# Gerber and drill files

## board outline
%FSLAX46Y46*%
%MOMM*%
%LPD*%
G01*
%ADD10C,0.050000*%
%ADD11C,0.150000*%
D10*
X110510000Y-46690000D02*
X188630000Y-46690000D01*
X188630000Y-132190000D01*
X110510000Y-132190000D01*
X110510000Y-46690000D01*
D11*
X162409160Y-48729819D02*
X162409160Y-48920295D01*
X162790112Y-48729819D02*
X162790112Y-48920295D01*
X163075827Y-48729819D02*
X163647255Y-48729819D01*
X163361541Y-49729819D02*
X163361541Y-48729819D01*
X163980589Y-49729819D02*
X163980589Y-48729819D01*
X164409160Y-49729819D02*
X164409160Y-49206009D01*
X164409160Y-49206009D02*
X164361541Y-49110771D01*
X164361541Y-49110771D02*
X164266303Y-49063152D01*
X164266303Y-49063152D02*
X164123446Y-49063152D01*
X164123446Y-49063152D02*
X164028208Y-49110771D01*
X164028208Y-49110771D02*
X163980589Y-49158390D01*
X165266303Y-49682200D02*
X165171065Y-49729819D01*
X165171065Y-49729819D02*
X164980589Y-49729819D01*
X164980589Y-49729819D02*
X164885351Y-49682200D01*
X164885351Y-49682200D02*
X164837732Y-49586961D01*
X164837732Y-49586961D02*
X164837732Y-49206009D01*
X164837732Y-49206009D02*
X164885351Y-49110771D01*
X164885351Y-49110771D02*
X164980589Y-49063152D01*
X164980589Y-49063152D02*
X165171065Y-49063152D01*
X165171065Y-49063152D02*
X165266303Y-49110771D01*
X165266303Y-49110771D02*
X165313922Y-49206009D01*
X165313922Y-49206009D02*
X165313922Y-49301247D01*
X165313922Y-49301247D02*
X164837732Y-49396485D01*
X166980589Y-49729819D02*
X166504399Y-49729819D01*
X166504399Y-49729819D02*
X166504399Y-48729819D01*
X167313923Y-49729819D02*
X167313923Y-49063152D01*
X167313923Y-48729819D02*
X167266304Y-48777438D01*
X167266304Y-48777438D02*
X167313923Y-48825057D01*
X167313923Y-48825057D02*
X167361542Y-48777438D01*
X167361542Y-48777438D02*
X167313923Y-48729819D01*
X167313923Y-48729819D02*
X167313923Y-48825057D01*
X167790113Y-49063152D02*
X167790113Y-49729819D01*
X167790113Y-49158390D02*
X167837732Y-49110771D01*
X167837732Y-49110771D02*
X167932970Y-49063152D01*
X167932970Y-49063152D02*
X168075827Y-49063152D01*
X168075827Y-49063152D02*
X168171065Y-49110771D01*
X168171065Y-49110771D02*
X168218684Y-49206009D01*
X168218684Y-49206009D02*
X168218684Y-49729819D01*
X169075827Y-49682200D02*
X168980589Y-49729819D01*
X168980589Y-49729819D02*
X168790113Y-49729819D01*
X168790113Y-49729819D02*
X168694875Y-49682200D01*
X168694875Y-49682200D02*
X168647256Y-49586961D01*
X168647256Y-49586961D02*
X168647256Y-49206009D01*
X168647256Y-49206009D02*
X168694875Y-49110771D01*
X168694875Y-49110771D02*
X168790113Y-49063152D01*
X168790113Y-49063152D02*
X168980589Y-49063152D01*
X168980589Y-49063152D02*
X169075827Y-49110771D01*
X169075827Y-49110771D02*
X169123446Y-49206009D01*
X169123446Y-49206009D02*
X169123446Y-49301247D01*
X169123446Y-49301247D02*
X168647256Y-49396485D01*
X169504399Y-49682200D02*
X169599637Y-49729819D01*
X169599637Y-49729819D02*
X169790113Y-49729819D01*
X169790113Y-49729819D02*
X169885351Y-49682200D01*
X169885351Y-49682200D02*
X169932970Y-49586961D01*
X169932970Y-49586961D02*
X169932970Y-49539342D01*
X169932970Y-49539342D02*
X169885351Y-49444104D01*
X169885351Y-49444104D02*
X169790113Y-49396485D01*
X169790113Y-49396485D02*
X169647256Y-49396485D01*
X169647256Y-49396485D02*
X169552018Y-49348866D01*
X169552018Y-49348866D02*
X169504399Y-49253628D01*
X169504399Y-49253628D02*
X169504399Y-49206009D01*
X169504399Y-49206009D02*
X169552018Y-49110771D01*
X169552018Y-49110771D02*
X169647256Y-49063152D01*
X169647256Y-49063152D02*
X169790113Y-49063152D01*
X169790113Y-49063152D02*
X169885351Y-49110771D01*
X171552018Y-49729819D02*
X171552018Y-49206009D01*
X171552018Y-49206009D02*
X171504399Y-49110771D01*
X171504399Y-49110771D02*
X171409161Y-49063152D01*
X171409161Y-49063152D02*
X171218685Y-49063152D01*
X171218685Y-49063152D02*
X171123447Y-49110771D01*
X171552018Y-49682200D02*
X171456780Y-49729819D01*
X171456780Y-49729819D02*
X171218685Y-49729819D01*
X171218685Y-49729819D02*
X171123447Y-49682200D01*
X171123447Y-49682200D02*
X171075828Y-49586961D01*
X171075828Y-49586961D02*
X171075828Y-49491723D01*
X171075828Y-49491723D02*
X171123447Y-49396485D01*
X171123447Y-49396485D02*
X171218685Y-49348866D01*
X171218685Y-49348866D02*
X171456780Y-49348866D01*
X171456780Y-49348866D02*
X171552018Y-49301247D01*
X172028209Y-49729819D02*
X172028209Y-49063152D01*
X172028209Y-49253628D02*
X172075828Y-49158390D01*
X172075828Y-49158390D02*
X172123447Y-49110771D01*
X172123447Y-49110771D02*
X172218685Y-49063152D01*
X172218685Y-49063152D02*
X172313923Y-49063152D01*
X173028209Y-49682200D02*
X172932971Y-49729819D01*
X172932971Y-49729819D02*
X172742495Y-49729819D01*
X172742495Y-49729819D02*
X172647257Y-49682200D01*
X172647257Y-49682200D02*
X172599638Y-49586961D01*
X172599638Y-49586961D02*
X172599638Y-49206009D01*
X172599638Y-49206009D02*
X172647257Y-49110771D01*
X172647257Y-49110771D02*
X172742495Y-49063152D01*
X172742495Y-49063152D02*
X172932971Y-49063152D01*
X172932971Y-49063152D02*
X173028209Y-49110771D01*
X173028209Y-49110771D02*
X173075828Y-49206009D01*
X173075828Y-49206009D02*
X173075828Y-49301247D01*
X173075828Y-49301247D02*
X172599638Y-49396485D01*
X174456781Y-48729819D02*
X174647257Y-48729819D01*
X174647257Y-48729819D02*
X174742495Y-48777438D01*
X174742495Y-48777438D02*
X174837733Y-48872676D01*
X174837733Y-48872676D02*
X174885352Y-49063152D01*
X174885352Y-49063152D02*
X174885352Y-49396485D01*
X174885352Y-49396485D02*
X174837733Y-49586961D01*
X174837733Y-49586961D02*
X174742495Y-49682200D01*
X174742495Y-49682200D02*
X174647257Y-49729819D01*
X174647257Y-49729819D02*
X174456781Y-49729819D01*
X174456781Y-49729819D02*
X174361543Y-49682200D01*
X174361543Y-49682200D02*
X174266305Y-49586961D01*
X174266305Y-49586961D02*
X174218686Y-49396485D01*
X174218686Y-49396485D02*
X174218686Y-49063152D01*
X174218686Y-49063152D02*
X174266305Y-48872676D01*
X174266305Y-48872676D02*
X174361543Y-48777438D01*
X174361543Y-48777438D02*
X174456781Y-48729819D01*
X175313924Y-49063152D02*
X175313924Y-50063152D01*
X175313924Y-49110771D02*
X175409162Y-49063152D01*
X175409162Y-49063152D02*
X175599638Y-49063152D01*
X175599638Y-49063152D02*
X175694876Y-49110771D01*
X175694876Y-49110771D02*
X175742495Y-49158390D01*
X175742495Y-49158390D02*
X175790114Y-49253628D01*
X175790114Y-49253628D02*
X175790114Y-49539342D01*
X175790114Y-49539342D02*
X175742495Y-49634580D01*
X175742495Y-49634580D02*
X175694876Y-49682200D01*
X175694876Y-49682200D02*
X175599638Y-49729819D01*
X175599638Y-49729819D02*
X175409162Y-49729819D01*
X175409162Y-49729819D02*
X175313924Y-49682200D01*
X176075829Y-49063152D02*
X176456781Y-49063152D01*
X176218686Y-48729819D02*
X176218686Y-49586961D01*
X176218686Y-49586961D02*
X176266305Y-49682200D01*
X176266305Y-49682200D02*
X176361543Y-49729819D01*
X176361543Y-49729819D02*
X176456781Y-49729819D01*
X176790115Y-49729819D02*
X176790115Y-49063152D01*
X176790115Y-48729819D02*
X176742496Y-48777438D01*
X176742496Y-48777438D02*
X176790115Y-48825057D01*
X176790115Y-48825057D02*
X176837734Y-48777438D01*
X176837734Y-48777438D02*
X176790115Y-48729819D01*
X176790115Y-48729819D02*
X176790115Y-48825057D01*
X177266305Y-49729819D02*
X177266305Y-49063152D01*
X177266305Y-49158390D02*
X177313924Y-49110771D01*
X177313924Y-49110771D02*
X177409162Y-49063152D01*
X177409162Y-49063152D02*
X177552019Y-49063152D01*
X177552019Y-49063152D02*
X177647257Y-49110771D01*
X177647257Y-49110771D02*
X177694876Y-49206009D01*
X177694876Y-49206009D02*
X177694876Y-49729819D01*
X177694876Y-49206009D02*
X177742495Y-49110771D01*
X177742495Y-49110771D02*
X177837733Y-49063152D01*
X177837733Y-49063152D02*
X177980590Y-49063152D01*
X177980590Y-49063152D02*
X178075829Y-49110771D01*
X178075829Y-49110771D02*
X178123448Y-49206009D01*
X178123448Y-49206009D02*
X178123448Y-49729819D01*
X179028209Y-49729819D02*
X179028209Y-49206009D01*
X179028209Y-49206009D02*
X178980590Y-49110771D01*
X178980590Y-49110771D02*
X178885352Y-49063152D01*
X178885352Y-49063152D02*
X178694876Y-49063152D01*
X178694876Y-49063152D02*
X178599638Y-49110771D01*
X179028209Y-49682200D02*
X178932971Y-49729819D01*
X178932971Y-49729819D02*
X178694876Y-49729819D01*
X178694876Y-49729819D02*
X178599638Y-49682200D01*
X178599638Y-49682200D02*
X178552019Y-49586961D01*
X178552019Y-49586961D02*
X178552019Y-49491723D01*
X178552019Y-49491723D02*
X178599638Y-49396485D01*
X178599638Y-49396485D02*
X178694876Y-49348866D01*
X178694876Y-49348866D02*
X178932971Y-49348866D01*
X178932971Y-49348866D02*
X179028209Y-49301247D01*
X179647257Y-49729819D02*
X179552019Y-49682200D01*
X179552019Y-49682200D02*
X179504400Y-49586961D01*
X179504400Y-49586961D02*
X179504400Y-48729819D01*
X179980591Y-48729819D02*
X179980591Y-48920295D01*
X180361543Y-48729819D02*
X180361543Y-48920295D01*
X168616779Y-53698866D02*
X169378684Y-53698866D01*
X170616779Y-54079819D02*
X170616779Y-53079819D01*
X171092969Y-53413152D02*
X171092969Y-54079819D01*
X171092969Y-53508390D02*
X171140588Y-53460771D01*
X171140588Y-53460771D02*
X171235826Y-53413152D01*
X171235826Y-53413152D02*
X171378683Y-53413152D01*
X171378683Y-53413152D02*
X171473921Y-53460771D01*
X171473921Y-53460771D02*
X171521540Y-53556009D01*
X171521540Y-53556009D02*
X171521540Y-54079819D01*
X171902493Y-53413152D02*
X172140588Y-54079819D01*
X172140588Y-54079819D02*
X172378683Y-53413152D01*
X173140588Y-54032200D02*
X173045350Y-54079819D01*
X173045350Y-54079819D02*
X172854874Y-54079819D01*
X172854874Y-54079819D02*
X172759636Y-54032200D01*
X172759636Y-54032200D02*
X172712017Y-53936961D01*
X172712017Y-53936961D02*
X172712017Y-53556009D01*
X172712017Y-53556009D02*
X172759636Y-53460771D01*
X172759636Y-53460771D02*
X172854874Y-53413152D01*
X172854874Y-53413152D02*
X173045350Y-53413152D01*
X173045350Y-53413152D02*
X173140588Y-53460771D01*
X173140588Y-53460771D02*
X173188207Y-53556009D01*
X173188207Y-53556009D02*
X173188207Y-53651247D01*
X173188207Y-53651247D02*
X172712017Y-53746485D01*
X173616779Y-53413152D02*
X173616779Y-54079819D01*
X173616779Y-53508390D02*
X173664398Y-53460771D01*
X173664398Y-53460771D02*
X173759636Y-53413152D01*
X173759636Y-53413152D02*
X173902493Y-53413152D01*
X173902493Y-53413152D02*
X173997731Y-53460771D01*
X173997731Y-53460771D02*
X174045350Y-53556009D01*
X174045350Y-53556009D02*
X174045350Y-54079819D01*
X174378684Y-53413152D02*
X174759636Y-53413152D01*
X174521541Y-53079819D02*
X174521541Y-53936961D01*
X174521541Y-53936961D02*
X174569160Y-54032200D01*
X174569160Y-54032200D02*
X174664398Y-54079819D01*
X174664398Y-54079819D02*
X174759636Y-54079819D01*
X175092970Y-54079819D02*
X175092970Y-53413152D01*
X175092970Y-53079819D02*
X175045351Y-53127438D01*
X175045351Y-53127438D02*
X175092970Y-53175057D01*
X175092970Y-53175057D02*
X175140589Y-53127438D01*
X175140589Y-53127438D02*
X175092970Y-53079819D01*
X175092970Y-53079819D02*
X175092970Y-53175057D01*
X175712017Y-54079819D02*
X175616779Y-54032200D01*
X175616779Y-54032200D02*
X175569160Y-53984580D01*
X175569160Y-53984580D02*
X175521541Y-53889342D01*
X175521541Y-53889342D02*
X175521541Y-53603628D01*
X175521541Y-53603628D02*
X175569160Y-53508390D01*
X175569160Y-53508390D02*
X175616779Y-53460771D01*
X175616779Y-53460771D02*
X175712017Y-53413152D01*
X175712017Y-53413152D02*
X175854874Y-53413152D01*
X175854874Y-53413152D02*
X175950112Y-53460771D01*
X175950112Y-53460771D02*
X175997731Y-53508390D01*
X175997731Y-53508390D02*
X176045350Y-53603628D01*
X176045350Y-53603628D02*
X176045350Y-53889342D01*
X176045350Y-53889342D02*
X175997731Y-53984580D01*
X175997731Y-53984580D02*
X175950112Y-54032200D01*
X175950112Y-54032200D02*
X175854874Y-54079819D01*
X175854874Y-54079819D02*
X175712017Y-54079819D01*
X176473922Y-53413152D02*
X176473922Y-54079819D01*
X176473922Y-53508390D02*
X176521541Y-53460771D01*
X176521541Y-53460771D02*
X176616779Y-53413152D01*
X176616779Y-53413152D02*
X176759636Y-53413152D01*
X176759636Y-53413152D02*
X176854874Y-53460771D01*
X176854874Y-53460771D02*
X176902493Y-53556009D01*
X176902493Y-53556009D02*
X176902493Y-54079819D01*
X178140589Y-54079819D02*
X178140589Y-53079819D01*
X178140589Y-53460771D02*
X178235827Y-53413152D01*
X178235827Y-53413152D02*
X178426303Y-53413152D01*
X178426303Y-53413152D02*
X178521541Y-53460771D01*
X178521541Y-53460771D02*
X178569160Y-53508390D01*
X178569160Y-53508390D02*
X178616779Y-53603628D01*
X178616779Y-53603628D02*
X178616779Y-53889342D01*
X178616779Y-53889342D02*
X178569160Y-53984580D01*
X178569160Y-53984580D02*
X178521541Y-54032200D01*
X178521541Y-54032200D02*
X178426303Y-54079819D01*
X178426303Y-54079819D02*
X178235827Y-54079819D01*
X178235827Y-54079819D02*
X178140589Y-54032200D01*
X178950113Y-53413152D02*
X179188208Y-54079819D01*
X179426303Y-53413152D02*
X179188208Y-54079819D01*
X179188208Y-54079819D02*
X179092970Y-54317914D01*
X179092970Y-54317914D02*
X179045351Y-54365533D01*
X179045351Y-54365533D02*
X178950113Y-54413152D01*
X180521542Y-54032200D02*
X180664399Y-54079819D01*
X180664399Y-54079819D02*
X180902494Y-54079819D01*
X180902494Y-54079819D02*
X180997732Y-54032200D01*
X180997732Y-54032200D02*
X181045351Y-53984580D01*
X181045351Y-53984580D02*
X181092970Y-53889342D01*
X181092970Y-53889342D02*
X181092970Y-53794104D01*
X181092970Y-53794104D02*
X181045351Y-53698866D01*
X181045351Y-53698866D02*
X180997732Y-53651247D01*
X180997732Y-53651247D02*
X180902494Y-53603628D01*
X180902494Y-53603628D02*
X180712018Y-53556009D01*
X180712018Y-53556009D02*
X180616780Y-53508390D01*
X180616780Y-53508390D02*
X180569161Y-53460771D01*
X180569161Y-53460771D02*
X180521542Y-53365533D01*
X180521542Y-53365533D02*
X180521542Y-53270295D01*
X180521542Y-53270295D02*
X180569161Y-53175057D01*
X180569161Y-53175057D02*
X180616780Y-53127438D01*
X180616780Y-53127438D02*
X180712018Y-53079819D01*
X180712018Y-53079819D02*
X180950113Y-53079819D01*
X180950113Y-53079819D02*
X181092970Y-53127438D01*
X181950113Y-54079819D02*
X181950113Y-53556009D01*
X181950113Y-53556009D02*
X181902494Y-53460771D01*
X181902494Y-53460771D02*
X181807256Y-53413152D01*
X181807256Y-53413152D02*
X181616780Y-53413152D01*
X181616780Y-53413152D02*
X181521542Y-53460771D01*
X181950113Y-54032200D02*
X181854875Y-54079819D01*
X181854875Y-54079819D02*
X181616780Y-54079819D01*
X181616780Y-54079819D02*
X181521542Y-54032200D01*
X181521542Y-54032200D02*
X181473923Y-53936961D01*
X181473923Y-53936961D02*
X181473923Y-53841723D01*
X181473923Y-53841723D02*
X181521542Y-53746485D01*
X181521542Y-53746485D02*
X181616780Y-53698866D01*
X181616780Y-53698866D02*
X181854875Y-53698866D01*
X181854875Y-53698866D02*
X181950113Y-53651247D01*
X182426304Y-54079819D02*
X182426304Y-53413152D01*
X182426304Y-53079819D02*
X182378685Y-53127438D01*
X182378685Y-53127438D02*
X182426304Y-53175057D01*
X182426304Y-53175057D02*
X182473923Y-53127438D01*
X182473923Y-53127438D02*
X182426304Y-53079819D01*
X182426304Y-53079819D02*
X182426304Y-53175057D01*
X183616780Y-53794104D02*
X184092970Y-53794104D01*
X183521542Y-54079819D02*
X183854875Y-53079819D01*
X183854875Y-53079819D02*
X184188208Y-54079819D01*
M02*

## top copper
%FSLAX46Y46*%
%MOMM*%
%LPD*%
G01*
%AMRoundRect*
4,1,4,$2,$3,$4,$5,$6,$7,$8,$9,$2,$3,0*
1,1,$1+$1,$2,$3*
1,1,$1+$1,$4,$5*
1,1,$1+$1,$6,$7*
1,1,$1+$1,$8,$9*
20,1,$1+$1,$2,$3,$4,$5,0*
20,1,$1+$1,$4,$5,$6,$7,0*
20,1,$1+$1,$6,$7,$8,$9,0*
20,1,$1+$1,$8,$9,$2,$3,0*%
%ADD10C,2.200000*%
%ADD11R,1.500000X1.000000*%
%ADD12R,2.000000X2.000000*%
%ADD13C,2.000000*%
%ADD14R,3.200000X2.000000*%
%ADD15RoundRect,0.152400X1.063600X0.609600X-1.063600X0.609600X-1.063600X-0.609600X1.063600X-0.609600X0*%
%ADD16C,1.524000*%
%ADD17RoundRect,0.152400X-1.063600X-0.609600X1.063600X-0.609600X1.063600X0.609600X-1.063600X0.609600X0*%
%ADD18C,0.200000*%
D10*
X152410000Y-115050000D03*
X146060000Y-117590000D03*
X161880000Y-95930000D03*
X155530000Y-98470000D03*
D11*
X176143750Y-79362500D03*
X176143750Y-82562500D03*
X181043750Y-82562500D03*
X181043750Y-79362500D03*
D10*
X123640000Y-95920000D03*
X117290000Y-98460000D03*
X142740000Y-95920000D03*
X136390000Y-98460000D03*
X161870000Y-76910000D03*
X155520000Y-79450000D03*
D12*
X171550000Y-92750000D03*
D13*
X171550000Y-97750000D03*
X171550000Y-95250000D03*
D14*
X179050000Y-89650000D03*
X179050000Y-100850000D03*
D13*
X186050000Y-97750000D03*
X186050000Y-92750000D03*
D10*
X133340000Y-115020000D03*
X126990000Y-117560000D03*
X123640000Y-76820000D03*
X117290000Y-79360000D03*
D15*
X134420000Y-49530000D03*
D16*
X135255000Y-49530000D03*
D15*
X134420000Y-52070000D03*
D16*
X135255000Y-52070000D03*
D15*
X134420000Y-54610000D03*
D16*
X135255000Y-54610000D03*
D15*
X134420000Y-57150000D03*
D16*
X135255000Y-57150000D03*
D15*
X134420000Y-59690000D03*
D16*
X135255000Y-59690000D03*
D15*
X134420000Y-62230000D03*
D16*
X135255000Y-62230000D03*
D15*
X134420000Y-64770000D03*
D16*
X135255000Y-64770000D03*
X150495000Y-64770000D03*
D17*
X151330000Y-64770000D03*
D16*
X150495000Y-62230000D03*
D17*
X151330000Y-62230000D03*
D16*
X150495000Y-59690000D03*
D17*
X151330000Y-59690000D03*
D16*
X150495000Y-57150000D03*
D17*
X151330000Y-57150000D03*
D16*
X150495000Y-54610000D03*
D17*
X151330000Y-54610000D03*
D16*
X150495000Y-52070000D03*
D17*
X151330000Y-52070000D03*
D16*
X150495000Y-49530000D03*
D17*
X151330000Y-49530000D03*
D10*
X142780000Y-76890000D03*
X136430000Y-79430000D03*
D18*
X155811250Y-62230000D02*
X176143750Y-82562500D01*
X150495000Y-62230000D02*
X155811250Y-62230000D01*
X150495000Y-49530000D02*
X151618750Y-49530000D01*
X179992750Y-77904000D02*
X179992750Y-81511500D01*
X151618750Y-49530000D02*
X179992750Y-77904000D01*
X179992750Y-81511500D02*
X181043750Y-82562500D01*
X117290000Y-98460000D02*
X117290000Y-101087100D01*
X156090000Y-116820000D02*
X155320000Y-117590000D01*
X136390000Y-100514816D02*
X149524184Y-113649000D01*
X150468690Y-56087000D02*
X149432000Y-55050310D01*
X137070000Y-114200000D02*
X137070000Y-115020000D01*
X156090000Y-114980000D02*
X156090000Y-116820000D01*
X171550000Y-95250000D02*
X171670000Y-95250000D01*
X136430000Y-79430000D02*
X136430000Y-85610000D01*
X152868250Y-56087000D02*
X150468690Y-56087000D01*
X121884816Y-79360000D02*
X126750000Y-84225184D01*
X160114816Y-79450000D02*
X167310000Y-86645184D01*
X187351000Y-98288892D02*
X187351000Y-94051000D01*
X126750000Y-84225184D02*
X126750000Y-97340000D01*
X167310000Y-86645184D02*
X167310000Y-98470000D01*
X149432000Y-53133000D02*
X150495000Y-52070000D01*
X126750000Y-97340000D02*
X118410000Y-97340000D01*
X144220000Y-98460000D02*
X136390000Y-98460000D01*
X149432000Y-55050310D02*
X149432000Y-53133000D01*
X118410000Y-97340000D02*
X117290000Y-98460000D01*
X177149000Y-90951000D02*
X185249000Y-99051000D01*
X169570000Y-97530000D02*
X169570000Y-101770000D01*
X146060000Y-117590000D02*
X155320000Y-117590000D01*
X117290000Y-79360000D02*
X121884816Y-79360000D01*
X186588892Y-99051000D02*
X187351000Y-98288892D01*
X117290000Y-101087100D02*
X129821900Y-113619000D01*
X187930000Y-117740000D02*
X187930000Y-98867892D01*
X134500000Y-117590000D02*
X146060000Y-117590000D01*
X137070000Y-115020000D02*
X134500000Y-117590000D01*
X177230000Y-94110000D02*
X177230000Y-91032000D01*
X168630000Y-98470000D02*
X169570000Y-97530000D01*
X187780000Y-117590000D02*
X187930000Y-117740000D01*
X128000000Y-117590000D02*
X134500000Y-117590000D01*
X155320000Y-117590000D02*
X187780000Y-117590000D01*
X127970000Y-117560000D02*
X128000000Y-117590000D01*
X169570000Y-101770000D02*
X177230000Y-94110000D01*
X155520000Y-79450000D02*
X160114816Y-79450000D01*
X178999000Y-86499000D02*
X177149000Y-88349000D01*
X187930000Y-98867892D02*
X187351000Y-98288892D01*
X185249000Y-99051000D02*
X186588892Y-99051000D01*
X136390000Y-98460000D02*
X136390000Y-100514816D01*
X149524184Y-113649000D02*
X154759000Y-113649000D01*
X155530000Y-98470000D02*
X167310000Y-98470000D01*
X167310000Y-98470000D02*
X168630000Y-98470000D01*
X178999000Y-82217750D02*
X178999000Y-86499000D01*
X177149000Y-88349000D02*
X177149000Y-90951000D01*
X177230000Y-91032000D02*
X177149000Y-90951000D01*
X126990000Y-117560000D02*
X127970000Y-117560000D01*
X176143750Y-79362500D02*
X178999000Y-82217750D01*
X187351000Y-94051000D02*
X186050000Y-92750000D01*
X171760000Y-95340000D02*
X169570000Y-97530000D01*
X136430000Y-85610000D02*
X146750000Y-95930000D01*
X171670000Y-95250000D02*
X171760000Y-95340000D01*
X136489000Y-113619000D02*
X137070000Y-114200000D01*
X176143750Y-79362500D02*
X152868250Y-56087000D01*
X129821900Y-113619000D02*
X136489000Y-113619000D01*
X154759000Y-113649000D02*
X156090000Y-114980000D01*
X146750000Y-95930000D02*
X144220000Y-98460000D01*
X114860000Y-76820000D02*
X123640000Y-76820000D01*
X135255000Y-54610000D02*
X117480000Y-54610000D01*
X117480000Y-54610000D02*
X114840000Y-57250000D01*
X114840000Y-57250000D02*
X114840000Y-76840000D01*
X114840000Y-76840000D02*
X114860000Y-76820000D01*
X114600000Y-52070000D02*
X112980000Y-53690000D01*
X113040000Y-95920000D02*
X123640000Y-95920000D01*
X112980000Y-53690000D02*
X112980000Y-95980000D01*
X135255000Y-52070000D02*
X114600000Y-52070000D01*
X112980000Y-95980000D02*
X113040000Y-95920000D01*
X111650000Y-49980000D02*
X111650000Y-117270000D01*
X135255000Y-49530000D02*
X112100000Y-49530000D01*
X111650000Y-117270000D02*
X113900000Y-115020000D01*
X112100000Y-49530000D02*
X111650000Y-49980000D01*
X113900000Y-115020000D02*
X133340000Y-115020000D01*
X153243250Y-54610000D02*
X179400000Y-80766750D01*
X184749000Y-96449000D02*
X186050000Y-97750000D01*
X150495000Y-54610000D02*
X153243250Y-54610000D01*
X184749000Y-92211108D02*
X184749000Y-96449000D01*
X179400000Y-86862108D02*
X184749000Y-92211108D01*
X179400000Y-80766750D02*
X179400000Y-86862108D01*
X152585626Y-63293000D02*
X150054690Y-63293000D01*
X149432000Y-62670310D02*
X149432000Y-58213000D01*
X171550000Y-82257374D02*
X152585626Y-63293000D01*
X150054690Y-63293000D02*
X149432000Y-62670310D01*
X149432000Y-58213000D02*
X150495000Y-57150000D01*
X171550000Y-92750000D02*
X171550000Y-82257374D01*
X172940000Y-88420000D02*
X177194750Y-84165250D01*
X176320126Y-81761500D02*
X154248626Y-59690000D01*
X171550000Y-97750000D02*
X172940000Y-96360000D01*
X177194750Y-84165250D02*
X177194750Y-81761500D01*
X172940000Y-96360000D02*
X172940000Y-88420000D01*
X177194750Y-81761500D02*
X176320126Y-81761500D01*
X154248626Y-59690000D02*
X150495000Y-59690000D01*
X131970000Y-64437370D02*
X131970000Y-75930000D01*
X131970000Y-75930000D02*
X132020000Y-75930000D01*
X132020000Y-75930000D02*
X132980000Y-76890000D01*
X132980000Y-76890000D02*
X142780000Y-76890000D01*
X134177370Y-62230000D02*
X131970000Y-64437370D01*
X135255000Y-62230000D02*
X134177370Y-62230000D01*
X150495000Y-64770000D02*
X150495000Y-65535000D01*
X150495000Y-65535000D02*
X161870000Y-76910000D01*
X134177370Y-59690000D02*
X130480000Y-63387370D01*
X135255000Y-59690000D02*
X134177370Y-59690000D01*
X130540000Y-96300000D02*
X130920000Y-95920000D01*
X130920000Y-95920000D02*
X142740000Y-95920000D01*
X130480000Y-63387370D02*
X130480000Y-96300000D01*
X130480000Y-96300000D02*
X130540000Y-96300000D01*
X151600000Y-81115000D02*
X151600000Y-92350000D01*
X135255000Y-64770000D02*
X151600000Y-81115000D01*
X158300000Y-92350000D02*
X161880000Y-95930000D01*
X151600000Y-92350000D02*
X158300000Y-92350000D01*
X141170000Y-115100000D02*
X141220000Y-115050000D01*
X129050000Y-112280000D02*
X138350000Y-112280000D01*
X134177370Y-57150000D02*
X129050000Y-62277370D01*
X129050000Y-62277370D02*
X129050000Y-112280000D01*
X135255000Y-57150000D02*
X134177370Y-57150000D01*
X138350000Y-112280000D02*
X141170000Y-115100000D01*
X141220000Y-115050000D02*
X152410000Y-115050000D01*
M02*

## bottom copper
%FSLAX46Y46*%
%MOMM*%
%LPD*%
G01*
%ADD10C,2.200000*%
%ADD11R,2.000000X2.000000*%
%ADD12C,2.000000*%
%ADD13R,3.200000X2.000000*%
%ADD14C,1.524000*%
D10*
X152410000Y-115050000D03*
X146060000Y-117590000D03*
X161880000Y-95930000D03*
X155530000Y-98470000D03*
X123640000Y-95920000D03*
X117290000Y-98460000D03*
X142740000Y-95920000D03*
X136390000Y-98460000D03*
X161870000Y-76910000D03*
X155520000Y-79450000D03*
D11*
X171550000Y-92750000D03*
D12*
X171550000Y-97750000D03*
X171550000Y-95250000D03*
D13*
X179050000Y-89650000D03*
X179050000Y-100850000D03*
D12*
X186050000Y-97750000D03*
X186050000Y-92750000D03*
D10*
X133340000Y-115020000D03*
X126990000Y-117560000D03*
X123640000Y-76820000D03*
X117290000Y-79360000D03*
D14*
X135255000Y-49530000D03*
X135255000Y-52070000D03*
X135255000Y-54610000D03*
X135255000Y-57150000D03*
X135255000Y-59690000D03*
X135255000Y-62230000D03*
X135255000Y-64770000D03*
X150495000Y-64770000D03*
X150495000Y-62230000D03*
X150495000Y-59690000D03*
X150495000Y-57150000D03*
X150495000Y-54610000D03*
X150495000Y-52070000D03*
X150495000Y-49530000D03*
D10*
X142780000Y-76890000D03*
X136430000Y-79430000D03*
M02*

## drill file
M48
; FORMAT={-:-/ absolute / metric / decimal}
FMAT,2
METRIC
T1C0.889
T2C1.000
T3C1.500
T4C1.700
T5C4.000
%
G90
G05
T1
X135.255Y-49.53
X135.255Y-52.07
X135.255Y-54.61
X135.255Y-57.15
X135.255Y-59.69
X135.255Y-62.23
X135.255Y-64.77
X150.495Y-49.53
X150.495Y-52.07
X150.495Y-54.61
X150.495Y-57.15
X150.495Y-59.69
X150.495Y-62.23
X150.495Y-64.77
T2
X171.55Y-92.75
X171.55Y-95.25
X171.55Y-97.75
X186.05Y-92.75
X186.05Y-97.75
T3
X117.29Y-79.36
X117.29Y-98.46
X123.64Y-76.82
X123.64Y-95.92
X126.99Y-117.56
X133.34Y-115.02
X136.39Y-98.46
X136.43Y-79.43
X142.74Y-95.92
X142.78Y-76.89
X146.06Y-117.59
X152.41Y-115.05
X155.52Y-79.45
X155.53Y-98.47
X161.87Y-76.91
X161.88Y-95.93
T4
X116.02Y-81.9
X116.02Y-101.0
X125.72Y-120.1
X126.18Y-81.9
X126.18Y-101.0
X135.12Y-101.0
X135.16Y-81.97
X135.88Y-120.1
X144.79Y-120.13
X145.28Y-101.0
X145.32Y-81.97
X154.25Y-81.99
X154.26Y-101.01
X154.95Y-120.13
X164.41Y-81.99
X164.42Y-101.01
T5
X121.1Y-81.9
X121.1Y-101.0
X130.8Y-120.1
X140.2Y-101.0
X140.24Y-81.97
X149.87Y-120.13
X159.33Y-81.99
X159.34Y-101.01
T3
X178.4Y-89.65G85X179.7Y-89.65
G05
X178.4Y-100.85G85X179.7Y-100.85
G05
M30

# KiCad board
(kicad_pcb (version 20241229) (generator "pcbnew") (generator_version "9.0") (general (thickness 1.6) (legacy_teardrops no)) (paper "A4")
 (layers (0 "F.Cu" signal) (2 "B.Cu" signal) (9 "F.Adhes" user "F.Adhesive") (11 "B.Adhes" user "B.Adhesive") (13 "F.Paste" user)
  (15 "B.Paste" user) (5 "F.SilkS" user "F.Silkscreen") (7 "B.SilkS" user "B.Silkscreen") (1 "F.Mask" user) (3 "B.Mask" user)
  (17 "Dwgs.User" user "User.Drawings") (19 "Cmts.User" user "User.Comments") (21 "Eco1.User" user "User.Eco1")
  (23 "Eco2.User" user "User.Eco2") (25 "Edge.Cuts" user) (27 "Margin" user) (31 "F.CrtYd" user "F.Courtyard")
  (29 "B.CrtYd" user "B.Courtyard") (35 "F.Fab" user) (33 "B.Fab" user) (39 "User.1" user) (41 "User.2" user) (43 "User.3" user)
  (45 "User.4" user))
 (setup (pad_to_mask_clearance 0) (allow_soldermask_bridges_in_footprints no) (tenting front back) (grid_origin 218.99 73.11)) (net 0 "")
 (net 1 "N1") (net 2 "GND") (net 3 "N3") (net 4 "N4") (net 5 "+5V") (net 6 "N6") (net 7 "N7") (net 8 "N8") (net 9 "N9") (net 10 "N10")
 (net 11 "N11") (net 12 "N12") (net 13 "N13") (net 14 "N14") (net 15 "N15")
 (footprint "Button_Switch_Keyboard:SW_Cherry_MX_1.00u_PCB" (layer "F.Cu") (at 152.41 115.05)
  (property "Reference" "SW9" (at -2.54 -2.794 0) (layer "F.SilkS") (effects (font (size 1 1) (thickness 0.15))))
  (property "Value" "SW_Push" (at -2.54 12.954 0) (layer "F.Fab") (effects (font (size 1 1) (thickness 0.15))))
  (pad "" np_thru_hole circle (at -7.62 5.08) (size 1.7 1.7) (drill 1.7) (layers "*.Cu" "*.Mask"))
  (pad "" np_thru_hole circle (at -2.54 5.08) (size 4 4) (drill 4) (layers "*.Cu" "*.Mask"))
  (pad "" np_thru_hole circle (at 2.54 5.08) (size 1.7 1.7) (drill 1.7) (layers "*.Cu" "*.Mask"))
  (pad "1" thru_hole circle (at 0 0) (size 2.2 2.2) (drill 1.5) (layers "*.Cu" "*.Mask") (remove_unused_layers no) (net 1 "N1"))
  (pad "2" thru_hole circle (at -6.35 2.54) (size 2.2 2.2) (drill 1.5) (layers "*.Cu" "*.Mask") (remove_unused_layers no) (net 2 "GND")))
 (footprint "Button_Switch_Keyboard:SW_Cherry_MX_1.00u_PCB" (layer "F.Cu") (at 161.88 95.93)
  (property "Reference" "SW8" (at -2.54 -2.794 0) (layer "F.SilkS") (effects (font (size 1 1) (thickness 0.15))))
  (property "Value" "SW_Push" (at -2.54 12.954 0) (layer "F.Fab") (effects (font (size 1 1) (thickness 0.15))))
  (pad "" np_thru_hole circle (at -7.62 5.08) (size 1.7 1.7) (drill 1.7) (layers "*.Cu" "*.Mask"))
  (pad "" np_thru_hole circle (at -2.54 5.08) (size 4 4) (drill 4) (layers "*.Cu" "*.Mask"))
  (pad "" np_thru_hole circle (at 2.54 5.08) (size 1.7 1.7) (drill 1.7) (layers "*.Cu" "*.Mask"))
  (pad "1" thru_hole circle (at 0 0) (size 2.2 2.2) (drill 1.5) (layers "*.Cu" "*.Mask") (remove_unused_layers no) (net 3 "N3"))
  (pad "2" thru_hole circle (at -6.35 2.54) (size 2.2 2.2) (drill 1.5) (layers "*.Cu" "*.Mask") (remove_unused_layers no) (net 2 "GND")))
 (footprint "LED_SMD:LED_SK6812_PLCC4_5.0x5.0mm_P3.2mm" (layer "F.Cu") (at 178.59375 80.9625)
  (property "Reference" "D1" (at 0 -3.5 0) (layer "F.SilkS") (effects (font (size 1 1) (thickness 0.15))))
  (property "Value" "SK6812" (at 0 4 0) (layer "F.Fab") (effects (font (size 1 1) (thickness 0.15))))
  (pad "1" smd rect (at -2.45 -1.6 180) (size 1.5 1) (layers "F.Cu" "F.Mask" "F.Paste") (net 2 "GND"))
  (pad "2" smd rect (at -2.45 1.6 180) (size 1.5 1) (layers "F.Cu" "F.Mask" "F.Paste") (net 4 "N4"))
  (pad "3" smd rect (at 2.45 1.6 180) (size 1.5 1) (layers "F.Cu" "F.Mask" "F.Paste") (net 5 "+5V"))
  (pad "4" smd rect (at 2.45 -1.6 180) (size 1.5 1) (layers "F.Cu" "F.Mask" "F.Paste") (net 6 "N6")))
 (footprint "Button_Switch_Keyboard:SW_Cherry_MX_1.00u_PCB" (layer "F.Cu") (at 123.64 95.92)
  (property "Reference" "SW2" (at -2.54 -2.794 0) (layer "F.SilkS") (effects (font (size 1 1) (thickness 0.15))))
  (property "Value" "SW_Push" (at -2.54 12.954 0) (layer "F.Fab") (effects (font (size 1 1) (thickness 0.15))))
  (pad "" np_thru_hole circle (at -7.62 5.08) (size 1.7 1.7) (drill 1.7) (layers "*.Cu" "*.Mask"))
  (pad "" np_thru_hole circle (at -2.54 5.08) (size 4 4) (drill 4) (layers "*.Cu" "*.Mask"))
  (pad "" np_thru_hole circle (at 2.54 5.08) (size 1.7 1.7) (drill 1.7) (layers "*.Cu" "*.Mask"))
  (pad "1" thru_hole circle (at 0 0) (size 2.2 2.2) (drill 1.5) (layers "*.Cu" "*.Mask") (remove_unused_layers no) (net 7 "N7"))
  (pad "2" thru_hole circle (at -6.35 2.54) (size 2.2 2.2) (drill 1.5) (layers "*.Cu" "*.Mask") (remove_unused_layers no) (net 2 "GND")))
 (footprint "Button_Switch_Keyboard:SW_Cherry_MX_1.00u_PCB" (layer "F.Cu") (at 142.74 95.92)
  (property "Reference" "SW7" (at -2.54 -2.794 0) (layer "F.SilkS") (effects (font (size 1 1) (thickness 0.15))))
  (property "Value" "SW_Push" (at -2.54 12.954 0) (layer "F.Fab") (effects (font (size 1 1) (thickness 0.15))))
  (pad "" np_thru_hole circle (at -7.62 5.08) (size 1.7 1.7) (drill 1.7) (layers "*.Cu" "*.Mask"))
  (pad "" np_thru_hole circle (at -2.54 5.08) (size 4 4) (drill 4) (layers "*.Cu" "*.Mask"))
  (pad "" np_thru_hole circle (at 2.54 5.08) (size 1.7 1.7) (drill 1.7) (layers "*.Cu" "*.Mask"))
  (pad "1" thru_hole circle (at 0 0) (size 2.2 2.2) (drill 1.5) (layers "*.Cu" "*.Mask") (remove_unused_layers no) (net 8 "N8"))
  (pad "2" thru_hole circle (at -6.35 2.54) (size 2.2 2.2) (drill 1.5) (layers "*.Cu" "*.Mask") (remove_unused_layers no) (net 2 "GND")))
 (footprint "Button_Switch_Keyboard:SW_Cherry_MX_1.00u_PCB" (layer "F.Cu") (at 161.87 76.91)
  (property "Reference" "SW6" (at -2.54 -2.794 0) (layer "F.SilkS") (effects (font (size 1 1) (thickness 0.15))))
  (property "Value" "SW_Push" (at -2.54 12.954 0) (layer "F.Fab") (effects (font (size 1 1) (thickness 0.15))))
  (pad "" np_thru_hole circle (at -7.62 5.08) (size 1.7 1.7) (drill 1.7) (layers "*.Cu" "*.Mask"))
  (pad "" np_thru_hole circle (at -2.54 5.08) (size 4 4) (drill 4) (layers "*.Cu" "*.Mask"))
  (pad "" np_thru_hole circle (at 2.54 5.08) (size 1.7 1.7) (drill 1.7) (layers "*.Cu" "*.Mask"))
  (pad "1" thru_hole circle (at 0 0) (size 2.2 2.2) (drill 1.5) (layers "*.Cu" "*.Mask") (remove_unused_layers no) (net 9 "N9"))
  (pad "2" thru_hole circle (at -6.35 2.54) (size 2.2 2.2) (drill 1.5) (layers "*.Cu" "*.Mask") (remove_unused_layers no) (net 2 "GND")))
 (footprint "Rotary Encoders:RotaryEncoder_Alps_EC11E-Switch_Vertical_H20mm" (layer "F.Cu") (at 171.55 92.75)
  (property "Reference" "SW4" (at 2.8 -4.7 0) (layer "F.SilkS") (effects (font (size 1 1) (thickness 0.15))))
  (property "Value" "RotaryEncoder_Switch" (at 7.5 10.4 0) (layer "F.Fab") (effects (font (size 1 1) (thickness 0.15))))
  (pad "A" thru_hole rect (at 0 0) (size 2 2) (drill 1) (layers "*.Cu" "*.Mask") (remove_unused_layers no) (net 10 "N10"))
  (pad "B" thru_hole circle (at 0 5) (size 2 2) (drill 1) (layers "*.Cu" "*.Mask") (remove_unused_layers no) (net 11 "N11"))
  (pad "C" thru_hole circle (at 0 2.5) (size 2 2) (drill 1) (layers "*.Cu" "*.Mask") (remove_unused_layers no) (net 2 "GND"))
  (pad "MP" thru_hole rect (at 7.5 -3.1) (size 3.2 2) (drill oval 2.8 1.5) (layers "*.Cu" "*.Mask") (remove_unused_layers no))
  (pad "MP" thru_hole rect (at 7.5 8.1) (size 3.2 2) (drill oval 2.8 1.5) (layers "*.Cu" "*.Mask") (remove_unused_layers no))
  (pad "S1" thru_hole circle (at 14.5 5) (size 2 2) (drill 1) (layers "*.Cu" "*.Mask") (remove_unused_layers no) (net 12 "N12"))
  (pad "S2" thru_hole circle (at 14.5 0) (size 2 2) (drill 1) (layers "*.Cu" "*.Mask") (remove_unused_layers no) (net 2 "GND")))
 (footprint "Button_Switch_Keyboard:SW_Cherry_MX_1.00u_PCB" (layer "F.Cu") (at 133.34 115.02)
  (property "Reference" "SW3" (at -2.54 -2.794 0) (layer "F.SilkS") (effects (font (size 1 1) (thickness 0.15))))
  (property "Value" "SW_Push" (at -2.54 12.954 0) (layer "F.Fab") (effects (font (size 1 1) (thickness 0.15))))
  (pad "" np_thru_hole circle (at -7.62 5.08) (size 1.7 1.7) (drill 1.7) (layers "*.Cu" "*.Mask"))
  (pad "" np_thru_hole circle (at -2.54 5.08) (size 4 4) (drill 4) (layers "*.Cu" "*.Mask"))
  (pad "" np_thru_hole circle (at 2.54 5.08) (size 1.7 1.7) (drill 1.7) (layers "*.Cu" "*.Mask"))
  (pad "1" thru_hole circle (at 0 0) (size 2.2 2.2) (drill 1.5) (layers "*.Cu" "*.Mask") (remove_unused_layers no) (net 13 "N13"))
  (pad "2" thru_hole circle (at -6.35 2.54) (size 2.2 2.2) (drill 1.5) (layers "*.Cu" "*.Mask") (remove_unused_layers no) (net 2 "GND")))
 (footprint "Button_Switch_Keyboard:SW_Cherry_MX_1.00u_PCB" (layer "F.Cu") (at 123.64 76.82)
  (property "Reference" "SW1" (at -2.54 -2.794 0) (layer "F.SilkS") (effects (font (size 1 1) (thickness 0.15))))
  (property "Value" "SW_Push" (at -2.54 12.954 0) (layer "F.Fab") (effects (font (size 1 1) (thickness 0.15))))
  (pad "" np_thru_hole circle (at -7.62 5.08) (size 1.7 1.7) (drill 1.7) (layers "*.Cu" "*.Mask"))
  (pad "" np_thru_hole circle (at -2.54 5.08) (size 4 4) (drill 4) (layers "*.Cu" "*.Mask"))
  (pad "" np_thru_hole circle (at 2.54 5.08) (size 1.7 1.7) (drill 1.7) (layers "*.Cu" "*.Mask"))
  (pad "1" thru_hole circle (at 0 0) (size 2.2 2.2) (drill 1.5) (layers "*.Cu" "*.Mask") (remove_unused_layers no) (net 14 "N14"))
  (pad "2" thru_hole circle (at -6.35 2.54) (size 2.2 2.2) (drill 1.5) (layers "*.Cu" "*.Mask") (remove_unused_layers no) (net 2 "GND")))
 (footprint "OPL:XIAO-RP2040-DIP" (layer "F.Cu") (at 142.875 57.15)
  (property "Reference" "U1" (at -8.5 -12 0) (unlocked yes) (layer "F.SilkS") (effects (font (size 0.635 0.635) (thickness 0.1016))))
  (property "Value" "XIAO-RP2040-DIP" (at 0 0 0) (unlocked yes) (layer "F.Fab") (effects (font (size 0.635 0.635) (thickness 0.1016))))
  (pad "1" smd roundrect (at -8.455 -7.62 180) (size 2.432 1.524) (layers "F.Cu" "F.Mask") (roundrect_rratio 0.1) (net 13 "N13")
   (thermal_bridge_angle 45))
  (pad "1" thru_hole circle (at -7.62 -7.62 180) (size 1.524 1.524) (drill 0.889) (layers "*.Cu" "*.Mask") (remove_unused_layers no)
   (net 13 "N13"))
  (pad "2" smd roundrect (at -8.455 -5.08 180) (size 2.432 1.524) (layers "F.Cu" "F.Mask") (roundrect_rratio 0.1) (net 7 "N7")
   (thermal_bridge_angle 45))
  (pad "2" thru_hole circle (at -7.62 -5.08 180) (size 1.524 1.524) (drill 0.889) (layers "*.Cu" "*.Mask") (remove_unused_layers no)
   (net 7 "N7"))
  (pad "3" smd roundrect (at -8.455 -2.54 180) (size 2.432 1.524) (layers "F.Cu" "F.Mask") (roundrect_rratio 0.1) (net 14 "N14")
   (thermal_bridge_angle 45))
  (pad "3" thru_hole circle (at -7.62 -2.54 180) (size 1.524 1.524) (drill 0.889) (layers "*.Cu" "*.Mask") (remove_unused_layers no)
   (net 14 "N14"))
  (pad "4" smd roundrect (at -8.455 0 180) (size 2.432 1.524) (layers "F.Cu" "F.Mask") (roundrect_rratio 0.1) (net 1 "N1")
   (thermal_bridge_angle 45))
  (pad "4" thru_hole circle (at -7.62 0 180) (size 1.524 1.524) (drill 0.889) (layers "*.Cu" "*.Mask") (remove_unused_layers no)
   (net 1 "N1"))
  (pad "5" smd roundrect (at -8.455 2.54 180) (size 2.432 1.524) (layers "F.Cu" "F.Mask") (roundrect_rratio 0.1) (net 8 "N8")
   (thermal_bridge_angle 45))
  (pad "5" thru_hole circle (at -7.62 2.54 180) (size 1.524 1.524) (drill 0.889) (layers "*.Cu" "*.Mask") (remove_unused_layers no)
   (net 8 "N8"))
  (pad "6" smd roundrect (at -8.455 5.08 180) (size 2.432 1.524) (layers "F.Cu" "F.Mask") (roundrect_rratio 0.1) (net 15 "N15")
   (thermal_bridge_angle 45))
  (pad "6" thru_hole circle (at -7.62 5.08 180) (size 1.524 1.524) (drill 0.889) (layers "*.Cu" "*.Mask") (remove_unused_layers no)
   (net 15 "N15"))
  (pad "7" smd roundrect (at -8.455 7.62 180) (size 2.432 1.524) (layers "F.Cu" "F.Mask") (roundrect_rratio 0.1) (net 3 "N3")
   (thermal_bridge_angle 45))
  (pad "7" thru_hole circle (at -7.62 7.62 180) (size 1.524 1.524) (drill 0.889) (layers "*.Cu" "*.Mask") (remove_unused_layers no)
   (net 3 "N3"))
  (pad "8" thru_hole circle (at 7.62 7.62) (size 1.524 1.524) (drill 0.889) (layers "*.Cu" "*.Mask") (remove_unused_layers no) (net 9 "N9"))
  (pad "8" smd roundrect (at 8.455 7.62) (size 2.432 1.524) (layers "F.Cu" "F.Mask") (roundrect_rratio 0.1) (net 9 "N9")
   (thermal_bridge_angle 45))
  (pad "9" thru_hole circle (at 7.62 5.08) (size 1.524 1.524) (drill 0.889) (layers "*.Cu" "*.Mask") (remove_unused_layers no) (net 4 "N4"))
  (pad "9" smd roundrect (at 8.455 5.08) (size 2.432 1.524) (layers "F.Cu" "F.Mask") (roundrect_rratio 0.1) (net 4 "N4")
   (thermal_bridge_angle 45))
  (pad "10" thru_hole circle (at 7.62 2.54) (size 1.524 1.524) (drill 0.889) (layers "*.Cu" "*.Mask") (remove_unused_layers no)
   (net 11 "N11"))
  (pad "10" smd roundrect (at 8.455 2.54) (size 2.432 1.524) (layers "F.Cu" "F.Mask") (roundrect_rratio 0.1) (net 11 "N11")
   (thermal_bridge_angle 45))
  (pad "11" thru_hole circle (at 7.62 0) (size 1.524 1.524) (drill 0.889) (layers "*.Cu" "*.Mask") (remove_unused_layers no) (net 10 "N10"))
  (pad "11" smd roundrect (at 8.455 0) (size 2.432 1.524) (layers "F.Cu" "F.Mask") (roundrect_rratio 0.1) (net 10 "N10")
   (thermal_bridge_angle 45))
  (pad "12" thru_hole circle (at 7.62 -2.54) (size 1.524 1.524) (drill 0.889) (layers "*.Cu" "*.Mask") (remove_unused_layers no)
   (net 12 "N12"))
  (pad "12" smd roundrect (at 8.455 -2.54) (size 2.432 1.524) (layers "F.Cu" "F.Mask") (roundrect_rratio 0.1) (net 12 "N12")
   (thermal_bridge_angle 45))
  (pad "13" thru_hole circle (at 7.62 -5.08) (size 1.524 1.524) (drill 0.889) (layers "*.Cu" "*.Mask") (remove_unused_layers no)
   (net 2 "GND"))
  (pad "13" smd roundrect (at 8.455 -5.08) (size 2.432 1.524) (layers "F.Cu" "F.Mask") (roundrect_rratio 0.1) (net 2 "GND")
   (thermal_bridge_angle 45))
  (pad "14" thru_hole circle (at 7.62 -7.62) (size 1.524 1.524) (drill 0.889) (layers "*.Cu" "*.Mask") (remove_unused_layers no)
   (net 5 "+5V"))
  (pad "14" smd roundrect (at 8.455 -7.62) (size 2.432 1.524) (layers "F.Cu" "F.Mask") (roundrect_rratio 0.1) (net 5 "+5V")
   (thermal_bridge_angle 45)))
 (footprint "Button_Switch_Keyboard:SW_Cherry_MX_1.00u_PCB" (layer "F.Cu") (at 142.78 76.89)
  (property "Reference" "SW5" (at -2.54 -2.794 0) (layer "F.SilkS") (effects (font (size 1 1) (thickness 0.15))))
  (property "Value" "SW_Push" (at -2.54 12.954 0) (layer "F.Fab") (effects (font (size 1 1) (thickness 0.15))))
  (pad "" np_thru_hole circle (at -7.62 5.08) (size 1.7 1.7) (drill 1.7) (layers "*.Cu" "*.Mask"))
  (pad "" np_thru_hole circle (at -2.54 5.08) (size 4 4) (drill 4) (layers "*.Cu" "*.Mask"))
  (pad "" np_thru_hole circle (at 2.54 5.08) (size 1.7 1.7) (drill 1.7) (layers "*.Cu" "*.Mask"))
  (pad "1" thru_hole circle (at 0 0) (size 2.2 2.2) (drill 1.5) (layers "*.Cu" "*.Mask") (remove_unused_layers no) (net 15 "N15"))
  (pad "2" thru_hole circle (at -6.35 2.54) (size 2.2 2.2) (drill 1.5) (layers "*.Cu" "*.Mask") (remove_unused_layers no) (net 2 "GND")))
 (gr_rect (start 110.51 46.69) (end 188.63 132.19) (stroke (width 0.05) (type default)) (fill no) (layer "Edge.Cuts"))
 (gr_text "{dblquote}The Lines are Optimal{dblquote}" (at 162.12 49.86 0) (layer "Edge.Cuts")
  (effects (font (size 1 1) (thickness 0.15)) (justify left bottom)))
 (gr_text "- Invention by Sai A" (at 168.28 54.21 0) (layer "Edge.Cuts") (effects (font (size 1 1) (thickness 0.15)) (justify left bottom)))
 (segment (start 155.81125 62.23) (end 176.14375 82.5625) (width 0.2) (layer "F.Cu") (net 4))
 (segment (start 150.495 62.23) (end 155.81125 62.23) (width 0.2) (layer "F.Cu") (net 4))
 (segment (start 150.495 49.53) (end 151.61875 49.53) (width 0.2) (layer "F.Cu") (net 5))
 (segment (start 179.99275 77.904) (end 179.99275 81.5115) (width 0.2) (layer "F.Cu") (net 5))
 (segment (start 151.61875 49.53) (end 179.99275 77.904) (width 0.2) (layer "F.Cu") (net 5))
 (segment (start 179.99275 81.5115) (end 181.04375 82.5625) (width 0.2) (layer "F.Cu") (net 5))
 (segment (start 117.29 98.46) (end 117.29 101.0871) (width 0.2) (layer "F.Cu") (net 2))
 (segment (start 156.09 116.82) (end 155.32 117.59) (width 0.2) (layer "F.Cu") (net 2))
 (segment (start 136.39 100.514816) (end 149.524184 113.649) (width 0.2) (layer "F.Cu") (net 2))
 (segment (start 150.46869 56.087) (end 149.432 55.05031) (width 0.2) (layer "F.Cu") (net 2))
 (segment (start 137.07 114.2) (end 137.07 115.02) (width 0.2) (layer "F.Cu") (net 2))
 (segment (start 156.09 114.98) (end 156.09 116.82) (width 0.2) (layer "F.Cu") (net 2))
 (segment (start 171.55 95.25) (end 171.67 95.25) (width 0.2) (layer "F.Cu") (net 2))
 (segment (start 136.43 79.43) (end 136.43 85.61) (width 0.2) (layer "F.Cu") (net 2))
 (segment (start 152.86825 56.087) (end 150.46869 56.087) (width 0.2) (layer "F.Cu") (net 2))
 (segment (start 121.884816 79.36) (end 126.75 84.225184) (width 0.2) (layer "F.Cu") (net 2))
 (segment (start 160.114816 79.45) (end 167.31 86.645184) (width 0.2) (layer "F.Cu") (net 2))
 (segment (start 187.351 98.288892) (end 187.351 94.051) (width 0.2) (layer "F.Cu") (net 2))
 (segment (start 126.75 84.225184) (end 126.75 97.34) (width 0.2) (layer "F.Cu") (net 2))
 (segment (start 167.31 86.645184) (end 167.31 98.47) (width 0.2) (layer "F.Cu") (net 2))
 (segment (start 149.432 53.133) (end 150.495 52.07) (width 0.2) (layer "F.Cu") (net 2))
 (segment (start 126.75 97.34) (end 118.41 97.34) (width 0.2) (layer "F.Cu") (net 2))
 (segment (start 144.22 98.46) (end 136.39 98.46) (width 0.2) (layer "F.Cu") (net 2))
 (segment (start 149.432 55.05031) (end 149.432 53.133) (width 0.2) (layer "F.Cu") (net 2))
 (segment (start 118.41 97.34) (end 117.29 98.46) (width 0.2) (layer "F.Cu") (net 2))
 (segment (start 177.149 90.951) (end 185.249 99.051) (width 0.2) (layer "F.Cu") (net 2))
 (segment (start 169.57 97.53) (end 169.57 101.77) (width 0.2) (layer "F.Cu") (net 2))
 (segment (start 146.06 117.59) (end 155.32 117.59) (width 0.2) (layer "F.Cu") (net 2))
 (segment (start 117.29 79.36) (end 121.884816 79.36) (width 0.2) (layer "F.Cu") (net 2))
 (segment (start 186.588892 99.051) (end 187.351 98.288892) (width 0.2) (layer "F.Cu") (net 2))
 (segment (start 117.29 101.0871) (end 129.8219 113.619) (width 0.2) (layer "F.Cu") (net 2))
 (segment (start 187.93 117.74) (end 187.93 98.867892) (width 0.2) (layer "F.Cu") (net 2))
 (segment (start 134.5 117.59) (end 146.06 117.59) (width 0.2) (layer "F.Cu") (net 2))
 (segment (start 137.07 115.02) (end 134.5 117.59) (width 0.2) (layer "F.Cu") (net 2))
 (segment (start 177.23 94.11) (end 177.23 91.032) (width 0.2) (layer "F.Cu") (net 2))
 (segment (start 168.63 98.47) (end 169.57 97.53) (width 0.2) (layer "F.Cu") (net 2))
 (segment (start 187.78 117.59) (end 187.93 117.74) (width 0.2) (layer "F.Cu") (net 2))
 (segment (start 128 117.59) (end 134.5 117.59) (width 0.2) (layer "F.Cu") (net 2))
 (segment (start 155.32 117.59) (end 187.78 117.59) (width 0.2) (layer "F.Cu") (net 2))
 (segment (start 127.97 117.56) (end 128 117.59) (width 0.2) (layer "F.Cu") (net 2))
 (segment (start 169.57 101.77) (end 177.23 94.11) (width 0.2) (layer "F.Cu") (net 2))
 (segment (start 155.52 79.45) (end 160.114816 79.45) (width 0.2) (layer "F.Cu") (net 2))
 (segment (start 178.999 86.499) (end 177.149 88.349) (width 0.2) (layer "F.Cu") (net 2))
 (segment (start 187.93 98.867892) (end 187.351 98.288892) (width 0.2) (layer "F.Cu") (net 2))
 (segment (start 185.249 99.051) (end 186.588892 99.051) (width 0.2) (layer "F.Cu") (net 2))
 (segment (start 136.39 98.46) (end 136.39 100.514816) (width 0.2) (layer "F.Cu") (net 2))
 (segment (start 149.524184 113.649) (end 154.759 113.649) (width 0.2) (layer "F.Cu") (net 2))
 (segment (start 155.53 98.47) (end 167.31 98.47) (width 0.2) (layer "F.Cu") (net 2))
 (segment (start 167.31 98.47) (end 168.63 98.47) (width 0.2) (layer "F.Cu") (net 2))
 (segment (start 178.999 82.21775) (end 178.999 86.499) (width 0.2) (layer "F.Cu") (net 2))
 (segment (start 177.149 88.349) (end 177.149 90.951) (width 0.2) (layer "F.Cu") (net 2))
 (segment (start 177.23 91.032) (end 177.149 90.951) (width 0.2) (layer "F.Cu") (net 2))
 (segment (start 126.99 117.56) (end 127.97 117.56) (width 0.2) (layer "F.Cu") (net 2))
 (segment (start 176.14375 79.3625) (end 178.999 82.21775) (width 0.2) (layer "F.Cu") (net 2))
 (segment (start 187.351 94.051) (end 186.05 92.75) (width 0.2) (layer "F.Cu") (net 2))
 (segment (start 171.76 95.34) (end 169.57 97.53) (width 0.2) (layer "F.Cu") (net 2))
 (segment (start 136.43 85.61) (end 146.75 95.93) (width 0.2) (layer "F.Cu") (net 2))
 (segment (start 171.67 95.25) (end 171.76 95.34) (width 0.2) (layer "F.Cu") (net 2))
 (segment (start 136.489 113.619) (end 137.07 114.2) (width 0.2) (layer "F.Cu") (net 2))
 (segment (start 176.14375 79.3625) (end 152.86825 56.087) (width 0.2) (layer "F.Cu") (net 2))
 (segment (start 129.8219 113.619) (end 136.489 113.619) (width 0.2) (layer "F.Cu") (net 2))
 (segment (start 154.759 113.649) (end 156.09 114.98) (width 0.2) (layer "F.Cu") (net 2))
 (segment (start 146.75 95.93) (end 144.22 98.46) (width 0.2) (layer "F.Cu") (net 2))
 (segment (start 114.86 76.82) (end 123.64 76.82) (width 0.2) (layer "F.Cu") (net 14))
 (segment (start 135.255 54.61) (end 117.48 54.61) (width 0.2) (layer "F.Cu") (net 14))
 (segment (start 117.48 54.61) (end 114.84 57.25) (width 0.2) (layer "F.Cu") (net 14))
 (segment (start 114.84 57.25) (end 114.84 76.84) (width 0.2) (layer "F.Cu") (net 14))
 (segment (start 114.84 76.84) (end 114.86 76.82) (width 0.2) (layer "F.Cu") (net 14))
 (segment (start 114.6 52.07) (end 112.98 53.69) (width 0.2) (layer "F.Cu") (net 7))
 (segment (start 113.04 95.92) (end 123.64 95.92) (width 0.2) (layer "F.Cu") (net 7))
 (segment (start 112.98 53.69) (end 112.98 95.98) (width 0.2) (layer "F.Cu") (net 7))
 (segment (start 135.255 52.07) (end 114.6 52.07) (width 0.2) (layer "F.Cu") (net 7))
 (segment (start 112.98 95.98) (end 113.04 95.92) (width 0.2) (layer "F.Cu") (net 7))
 (segment (start 111.65 49.98) (end 111.65 117.27) (width 0.2) (layer "F.Cu") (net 13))
 (segment (start 135.255 49.53) (end 112.1 49.53) (width 0.2) (layer "F.Cu") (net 13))
 (segment (start 111.65 117.27) (end 113.9 115.02) (width 0.2) (layer "F.Cu") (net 13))
 (segment (start 112.1 49.53) (end 111.65 49.98) (width 0.2) (layer "F.Cu") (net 13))
 (segment (start 113.9 115.02) (end 133.34 115.02) (width 0.2) (layer "F.Cu") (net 13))
 (segment (start 153.24325 54.61) (end 179.4 80.76675) (width 0.2) (layer "F.Cu") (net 12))
 (segment (start 184.749 96.449) (end 186.05 97.75) (width 0.2) (layer "F.Cu") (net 12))
 (segment (start 150.495 54.61) (end 153.24325 54.61) (width 0.2) (layer "F.Cu") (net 12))
 (segment (start 184.749 92.211108) (end 184.749 96.449) (width 0.2) (layer "F.Cu") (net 12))
 (segment (start 179.4 86.862108) (end 184.749 92.211108) (width 0.2) (layer "F.Cu") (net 12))
 (segment (start 179.4 80.76675) (end 179.4 86.862108) (width 0.2) (layer "F.Cu") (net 12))
 (segment (start 152.585626 63.293) (end 150.05469 63.293) (width 0.2) (layer "F.Cu") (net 10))
 (segment (start 149.432 62.67031) (end 149.432 58.213) (width 0.2) (layer "F.Cu") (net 10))
 (segment (start 171.55 82.257374) (end 152.585626 63.293) (width 0.2) (layer "F.Cu") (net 10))
 (segment (start 150.05469 63.293) (end 149.432 62.67031) (width 0.2) (layer "F.Cu") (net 10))
 (segment (start 149.432 58.213) (end 150.495 57.15) (width 0.2) (layer "F.Cu") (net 10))
 (segment (start 171.55 92.75) (end 171.55 82.257374) (width 0.2) (layer "F.Cu") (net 10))
 (segment (start 172.94 88.42) (end 177.19475 84.16525) (width 0.2) (layer "F.Cu") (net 11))
 (segment (start 176.320126 81.7615) (end 154.248626 59.69) (width 0.2) (layer "F.Cu") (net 11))
 (segment (start 171.55 97.75) (end 172.94 96.36) (width 0.2) (layer "F.Cu") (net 11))
 (segment (start 177.19475 84.16525) (end 177.19475 81.7615) (width 0.2) (layer "F.Cu") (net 11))
 (segment (start 172.94 96.36) (end 172.94 88.42) (width 0.2) (layer "F.Cu") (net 11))
 (segment (start 177.19475 81.7615) (end 176.320126 81.7615) (width 0.2) (layer "F.Cu") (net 11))
 (segment (start 154.248626 59.69) (end 150.495 59.69) (width 0.2) (layer "F.Cu") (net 11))
 (segment (start 131.97 64.43737) (end 131.97 75.93) (width 0.2) (layer "F.Cu") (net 15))
 (segment (start 131.97 75.93) (end 132.02 75.93) (width 0.2) (layer "F.Cu") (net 15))
 (segment (start 132.02 75.93) (end 132.98 76.89) (width 0.2) (layer "F.Cu") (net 15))
 (segment (start 132.98 76.89) (end 142.78 76.89) (width 0.2) (layer "F.Cu") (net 15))
 (segment (start 134.17737 62.23) (end 131.97 64.43737) (width 0.2) (layer "F.Cu") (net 15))
 (segment (start 135.255 62.23) (end 134.17737 62.23) (width 0.2) (layer "F.Cu") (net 15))
 (segment (start 150.495 64.77) (end 150.495 65.535) (width 0.2) (layer "F.Cu") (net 9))
 (segment (start 150.495 65.535) (end 161.87 76.91) (width 0.2) (layer "F.Cu") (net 9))
 (segment (start 134.17737 59.69) (end 130.48 63.38737) (width 0.2) (layer "F.Cu") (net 8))
 (segment (start 135.255 59.69) (end 134.17737 59.69) (width 0.2) (layer "F.Cu") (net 8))
 (segment (start 130.54 96.3) (end 130.92 95.92) (width 0.2) (layer "F.Cu") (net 8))
 (segment (start 130.92 95.92) (end 142.74 95.92) (width 0.2) (layer "F.Cu") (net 8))
 (segment (start 130.48 63.38737) (end 130.48 96.3) (width 0.2) (layer "F.Cu") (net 8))
 (segment (start 130.48 96.3) (end 130.54 96.3) (width 0.2) (layer "F.Cu") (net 8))
 (segment (start 151.6 81.115) (end 151.6 92.35) (width 0.2) (layer "F.Cu") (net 3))
 (segment (start 135.255 64.77) (end 151.6 81.115) (width 0.2) (layer "F.Cu") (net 3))
 (segment (start 158.3 92.35) (end 161.88 95.93) (width 0.2) (layer "F.Cu") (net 3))
 (segment (start 151.6 92.35) (end 158.3 92.35) (width 0.2) (layer "F.Cu") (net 3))
 (segment (start 141.17 115.1) (end 141.22 115.05) (width 0.2) (layer "F.Cu") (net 1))
 (segment (start 129.05 112.28) (end 138.35 112.28) (width 0.2) (layer "F.Cu") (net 1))
 (segment (start 134.17737 57.15) (end 129.05 62.27737) (width 0.2) (layer "F.Cu") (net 1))
 (segment (start 129.05 62.27737) (end 129.05 112.28) (width 0.2) (layer "F.Cu") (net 1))
 (segment (start 135.255 57.15) (end 134.17737 57.15) (width 0.2) (layer "F.Cu") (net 1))
 (segment (start 138.35 112.28) (end 141.17 115.1) (width 0.2) (layer "F.Cu") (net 1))
 (segment (start 141.22 115.05) (end 152.41 115.05) (width 0.2) (layer "F.Cu") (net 1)))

